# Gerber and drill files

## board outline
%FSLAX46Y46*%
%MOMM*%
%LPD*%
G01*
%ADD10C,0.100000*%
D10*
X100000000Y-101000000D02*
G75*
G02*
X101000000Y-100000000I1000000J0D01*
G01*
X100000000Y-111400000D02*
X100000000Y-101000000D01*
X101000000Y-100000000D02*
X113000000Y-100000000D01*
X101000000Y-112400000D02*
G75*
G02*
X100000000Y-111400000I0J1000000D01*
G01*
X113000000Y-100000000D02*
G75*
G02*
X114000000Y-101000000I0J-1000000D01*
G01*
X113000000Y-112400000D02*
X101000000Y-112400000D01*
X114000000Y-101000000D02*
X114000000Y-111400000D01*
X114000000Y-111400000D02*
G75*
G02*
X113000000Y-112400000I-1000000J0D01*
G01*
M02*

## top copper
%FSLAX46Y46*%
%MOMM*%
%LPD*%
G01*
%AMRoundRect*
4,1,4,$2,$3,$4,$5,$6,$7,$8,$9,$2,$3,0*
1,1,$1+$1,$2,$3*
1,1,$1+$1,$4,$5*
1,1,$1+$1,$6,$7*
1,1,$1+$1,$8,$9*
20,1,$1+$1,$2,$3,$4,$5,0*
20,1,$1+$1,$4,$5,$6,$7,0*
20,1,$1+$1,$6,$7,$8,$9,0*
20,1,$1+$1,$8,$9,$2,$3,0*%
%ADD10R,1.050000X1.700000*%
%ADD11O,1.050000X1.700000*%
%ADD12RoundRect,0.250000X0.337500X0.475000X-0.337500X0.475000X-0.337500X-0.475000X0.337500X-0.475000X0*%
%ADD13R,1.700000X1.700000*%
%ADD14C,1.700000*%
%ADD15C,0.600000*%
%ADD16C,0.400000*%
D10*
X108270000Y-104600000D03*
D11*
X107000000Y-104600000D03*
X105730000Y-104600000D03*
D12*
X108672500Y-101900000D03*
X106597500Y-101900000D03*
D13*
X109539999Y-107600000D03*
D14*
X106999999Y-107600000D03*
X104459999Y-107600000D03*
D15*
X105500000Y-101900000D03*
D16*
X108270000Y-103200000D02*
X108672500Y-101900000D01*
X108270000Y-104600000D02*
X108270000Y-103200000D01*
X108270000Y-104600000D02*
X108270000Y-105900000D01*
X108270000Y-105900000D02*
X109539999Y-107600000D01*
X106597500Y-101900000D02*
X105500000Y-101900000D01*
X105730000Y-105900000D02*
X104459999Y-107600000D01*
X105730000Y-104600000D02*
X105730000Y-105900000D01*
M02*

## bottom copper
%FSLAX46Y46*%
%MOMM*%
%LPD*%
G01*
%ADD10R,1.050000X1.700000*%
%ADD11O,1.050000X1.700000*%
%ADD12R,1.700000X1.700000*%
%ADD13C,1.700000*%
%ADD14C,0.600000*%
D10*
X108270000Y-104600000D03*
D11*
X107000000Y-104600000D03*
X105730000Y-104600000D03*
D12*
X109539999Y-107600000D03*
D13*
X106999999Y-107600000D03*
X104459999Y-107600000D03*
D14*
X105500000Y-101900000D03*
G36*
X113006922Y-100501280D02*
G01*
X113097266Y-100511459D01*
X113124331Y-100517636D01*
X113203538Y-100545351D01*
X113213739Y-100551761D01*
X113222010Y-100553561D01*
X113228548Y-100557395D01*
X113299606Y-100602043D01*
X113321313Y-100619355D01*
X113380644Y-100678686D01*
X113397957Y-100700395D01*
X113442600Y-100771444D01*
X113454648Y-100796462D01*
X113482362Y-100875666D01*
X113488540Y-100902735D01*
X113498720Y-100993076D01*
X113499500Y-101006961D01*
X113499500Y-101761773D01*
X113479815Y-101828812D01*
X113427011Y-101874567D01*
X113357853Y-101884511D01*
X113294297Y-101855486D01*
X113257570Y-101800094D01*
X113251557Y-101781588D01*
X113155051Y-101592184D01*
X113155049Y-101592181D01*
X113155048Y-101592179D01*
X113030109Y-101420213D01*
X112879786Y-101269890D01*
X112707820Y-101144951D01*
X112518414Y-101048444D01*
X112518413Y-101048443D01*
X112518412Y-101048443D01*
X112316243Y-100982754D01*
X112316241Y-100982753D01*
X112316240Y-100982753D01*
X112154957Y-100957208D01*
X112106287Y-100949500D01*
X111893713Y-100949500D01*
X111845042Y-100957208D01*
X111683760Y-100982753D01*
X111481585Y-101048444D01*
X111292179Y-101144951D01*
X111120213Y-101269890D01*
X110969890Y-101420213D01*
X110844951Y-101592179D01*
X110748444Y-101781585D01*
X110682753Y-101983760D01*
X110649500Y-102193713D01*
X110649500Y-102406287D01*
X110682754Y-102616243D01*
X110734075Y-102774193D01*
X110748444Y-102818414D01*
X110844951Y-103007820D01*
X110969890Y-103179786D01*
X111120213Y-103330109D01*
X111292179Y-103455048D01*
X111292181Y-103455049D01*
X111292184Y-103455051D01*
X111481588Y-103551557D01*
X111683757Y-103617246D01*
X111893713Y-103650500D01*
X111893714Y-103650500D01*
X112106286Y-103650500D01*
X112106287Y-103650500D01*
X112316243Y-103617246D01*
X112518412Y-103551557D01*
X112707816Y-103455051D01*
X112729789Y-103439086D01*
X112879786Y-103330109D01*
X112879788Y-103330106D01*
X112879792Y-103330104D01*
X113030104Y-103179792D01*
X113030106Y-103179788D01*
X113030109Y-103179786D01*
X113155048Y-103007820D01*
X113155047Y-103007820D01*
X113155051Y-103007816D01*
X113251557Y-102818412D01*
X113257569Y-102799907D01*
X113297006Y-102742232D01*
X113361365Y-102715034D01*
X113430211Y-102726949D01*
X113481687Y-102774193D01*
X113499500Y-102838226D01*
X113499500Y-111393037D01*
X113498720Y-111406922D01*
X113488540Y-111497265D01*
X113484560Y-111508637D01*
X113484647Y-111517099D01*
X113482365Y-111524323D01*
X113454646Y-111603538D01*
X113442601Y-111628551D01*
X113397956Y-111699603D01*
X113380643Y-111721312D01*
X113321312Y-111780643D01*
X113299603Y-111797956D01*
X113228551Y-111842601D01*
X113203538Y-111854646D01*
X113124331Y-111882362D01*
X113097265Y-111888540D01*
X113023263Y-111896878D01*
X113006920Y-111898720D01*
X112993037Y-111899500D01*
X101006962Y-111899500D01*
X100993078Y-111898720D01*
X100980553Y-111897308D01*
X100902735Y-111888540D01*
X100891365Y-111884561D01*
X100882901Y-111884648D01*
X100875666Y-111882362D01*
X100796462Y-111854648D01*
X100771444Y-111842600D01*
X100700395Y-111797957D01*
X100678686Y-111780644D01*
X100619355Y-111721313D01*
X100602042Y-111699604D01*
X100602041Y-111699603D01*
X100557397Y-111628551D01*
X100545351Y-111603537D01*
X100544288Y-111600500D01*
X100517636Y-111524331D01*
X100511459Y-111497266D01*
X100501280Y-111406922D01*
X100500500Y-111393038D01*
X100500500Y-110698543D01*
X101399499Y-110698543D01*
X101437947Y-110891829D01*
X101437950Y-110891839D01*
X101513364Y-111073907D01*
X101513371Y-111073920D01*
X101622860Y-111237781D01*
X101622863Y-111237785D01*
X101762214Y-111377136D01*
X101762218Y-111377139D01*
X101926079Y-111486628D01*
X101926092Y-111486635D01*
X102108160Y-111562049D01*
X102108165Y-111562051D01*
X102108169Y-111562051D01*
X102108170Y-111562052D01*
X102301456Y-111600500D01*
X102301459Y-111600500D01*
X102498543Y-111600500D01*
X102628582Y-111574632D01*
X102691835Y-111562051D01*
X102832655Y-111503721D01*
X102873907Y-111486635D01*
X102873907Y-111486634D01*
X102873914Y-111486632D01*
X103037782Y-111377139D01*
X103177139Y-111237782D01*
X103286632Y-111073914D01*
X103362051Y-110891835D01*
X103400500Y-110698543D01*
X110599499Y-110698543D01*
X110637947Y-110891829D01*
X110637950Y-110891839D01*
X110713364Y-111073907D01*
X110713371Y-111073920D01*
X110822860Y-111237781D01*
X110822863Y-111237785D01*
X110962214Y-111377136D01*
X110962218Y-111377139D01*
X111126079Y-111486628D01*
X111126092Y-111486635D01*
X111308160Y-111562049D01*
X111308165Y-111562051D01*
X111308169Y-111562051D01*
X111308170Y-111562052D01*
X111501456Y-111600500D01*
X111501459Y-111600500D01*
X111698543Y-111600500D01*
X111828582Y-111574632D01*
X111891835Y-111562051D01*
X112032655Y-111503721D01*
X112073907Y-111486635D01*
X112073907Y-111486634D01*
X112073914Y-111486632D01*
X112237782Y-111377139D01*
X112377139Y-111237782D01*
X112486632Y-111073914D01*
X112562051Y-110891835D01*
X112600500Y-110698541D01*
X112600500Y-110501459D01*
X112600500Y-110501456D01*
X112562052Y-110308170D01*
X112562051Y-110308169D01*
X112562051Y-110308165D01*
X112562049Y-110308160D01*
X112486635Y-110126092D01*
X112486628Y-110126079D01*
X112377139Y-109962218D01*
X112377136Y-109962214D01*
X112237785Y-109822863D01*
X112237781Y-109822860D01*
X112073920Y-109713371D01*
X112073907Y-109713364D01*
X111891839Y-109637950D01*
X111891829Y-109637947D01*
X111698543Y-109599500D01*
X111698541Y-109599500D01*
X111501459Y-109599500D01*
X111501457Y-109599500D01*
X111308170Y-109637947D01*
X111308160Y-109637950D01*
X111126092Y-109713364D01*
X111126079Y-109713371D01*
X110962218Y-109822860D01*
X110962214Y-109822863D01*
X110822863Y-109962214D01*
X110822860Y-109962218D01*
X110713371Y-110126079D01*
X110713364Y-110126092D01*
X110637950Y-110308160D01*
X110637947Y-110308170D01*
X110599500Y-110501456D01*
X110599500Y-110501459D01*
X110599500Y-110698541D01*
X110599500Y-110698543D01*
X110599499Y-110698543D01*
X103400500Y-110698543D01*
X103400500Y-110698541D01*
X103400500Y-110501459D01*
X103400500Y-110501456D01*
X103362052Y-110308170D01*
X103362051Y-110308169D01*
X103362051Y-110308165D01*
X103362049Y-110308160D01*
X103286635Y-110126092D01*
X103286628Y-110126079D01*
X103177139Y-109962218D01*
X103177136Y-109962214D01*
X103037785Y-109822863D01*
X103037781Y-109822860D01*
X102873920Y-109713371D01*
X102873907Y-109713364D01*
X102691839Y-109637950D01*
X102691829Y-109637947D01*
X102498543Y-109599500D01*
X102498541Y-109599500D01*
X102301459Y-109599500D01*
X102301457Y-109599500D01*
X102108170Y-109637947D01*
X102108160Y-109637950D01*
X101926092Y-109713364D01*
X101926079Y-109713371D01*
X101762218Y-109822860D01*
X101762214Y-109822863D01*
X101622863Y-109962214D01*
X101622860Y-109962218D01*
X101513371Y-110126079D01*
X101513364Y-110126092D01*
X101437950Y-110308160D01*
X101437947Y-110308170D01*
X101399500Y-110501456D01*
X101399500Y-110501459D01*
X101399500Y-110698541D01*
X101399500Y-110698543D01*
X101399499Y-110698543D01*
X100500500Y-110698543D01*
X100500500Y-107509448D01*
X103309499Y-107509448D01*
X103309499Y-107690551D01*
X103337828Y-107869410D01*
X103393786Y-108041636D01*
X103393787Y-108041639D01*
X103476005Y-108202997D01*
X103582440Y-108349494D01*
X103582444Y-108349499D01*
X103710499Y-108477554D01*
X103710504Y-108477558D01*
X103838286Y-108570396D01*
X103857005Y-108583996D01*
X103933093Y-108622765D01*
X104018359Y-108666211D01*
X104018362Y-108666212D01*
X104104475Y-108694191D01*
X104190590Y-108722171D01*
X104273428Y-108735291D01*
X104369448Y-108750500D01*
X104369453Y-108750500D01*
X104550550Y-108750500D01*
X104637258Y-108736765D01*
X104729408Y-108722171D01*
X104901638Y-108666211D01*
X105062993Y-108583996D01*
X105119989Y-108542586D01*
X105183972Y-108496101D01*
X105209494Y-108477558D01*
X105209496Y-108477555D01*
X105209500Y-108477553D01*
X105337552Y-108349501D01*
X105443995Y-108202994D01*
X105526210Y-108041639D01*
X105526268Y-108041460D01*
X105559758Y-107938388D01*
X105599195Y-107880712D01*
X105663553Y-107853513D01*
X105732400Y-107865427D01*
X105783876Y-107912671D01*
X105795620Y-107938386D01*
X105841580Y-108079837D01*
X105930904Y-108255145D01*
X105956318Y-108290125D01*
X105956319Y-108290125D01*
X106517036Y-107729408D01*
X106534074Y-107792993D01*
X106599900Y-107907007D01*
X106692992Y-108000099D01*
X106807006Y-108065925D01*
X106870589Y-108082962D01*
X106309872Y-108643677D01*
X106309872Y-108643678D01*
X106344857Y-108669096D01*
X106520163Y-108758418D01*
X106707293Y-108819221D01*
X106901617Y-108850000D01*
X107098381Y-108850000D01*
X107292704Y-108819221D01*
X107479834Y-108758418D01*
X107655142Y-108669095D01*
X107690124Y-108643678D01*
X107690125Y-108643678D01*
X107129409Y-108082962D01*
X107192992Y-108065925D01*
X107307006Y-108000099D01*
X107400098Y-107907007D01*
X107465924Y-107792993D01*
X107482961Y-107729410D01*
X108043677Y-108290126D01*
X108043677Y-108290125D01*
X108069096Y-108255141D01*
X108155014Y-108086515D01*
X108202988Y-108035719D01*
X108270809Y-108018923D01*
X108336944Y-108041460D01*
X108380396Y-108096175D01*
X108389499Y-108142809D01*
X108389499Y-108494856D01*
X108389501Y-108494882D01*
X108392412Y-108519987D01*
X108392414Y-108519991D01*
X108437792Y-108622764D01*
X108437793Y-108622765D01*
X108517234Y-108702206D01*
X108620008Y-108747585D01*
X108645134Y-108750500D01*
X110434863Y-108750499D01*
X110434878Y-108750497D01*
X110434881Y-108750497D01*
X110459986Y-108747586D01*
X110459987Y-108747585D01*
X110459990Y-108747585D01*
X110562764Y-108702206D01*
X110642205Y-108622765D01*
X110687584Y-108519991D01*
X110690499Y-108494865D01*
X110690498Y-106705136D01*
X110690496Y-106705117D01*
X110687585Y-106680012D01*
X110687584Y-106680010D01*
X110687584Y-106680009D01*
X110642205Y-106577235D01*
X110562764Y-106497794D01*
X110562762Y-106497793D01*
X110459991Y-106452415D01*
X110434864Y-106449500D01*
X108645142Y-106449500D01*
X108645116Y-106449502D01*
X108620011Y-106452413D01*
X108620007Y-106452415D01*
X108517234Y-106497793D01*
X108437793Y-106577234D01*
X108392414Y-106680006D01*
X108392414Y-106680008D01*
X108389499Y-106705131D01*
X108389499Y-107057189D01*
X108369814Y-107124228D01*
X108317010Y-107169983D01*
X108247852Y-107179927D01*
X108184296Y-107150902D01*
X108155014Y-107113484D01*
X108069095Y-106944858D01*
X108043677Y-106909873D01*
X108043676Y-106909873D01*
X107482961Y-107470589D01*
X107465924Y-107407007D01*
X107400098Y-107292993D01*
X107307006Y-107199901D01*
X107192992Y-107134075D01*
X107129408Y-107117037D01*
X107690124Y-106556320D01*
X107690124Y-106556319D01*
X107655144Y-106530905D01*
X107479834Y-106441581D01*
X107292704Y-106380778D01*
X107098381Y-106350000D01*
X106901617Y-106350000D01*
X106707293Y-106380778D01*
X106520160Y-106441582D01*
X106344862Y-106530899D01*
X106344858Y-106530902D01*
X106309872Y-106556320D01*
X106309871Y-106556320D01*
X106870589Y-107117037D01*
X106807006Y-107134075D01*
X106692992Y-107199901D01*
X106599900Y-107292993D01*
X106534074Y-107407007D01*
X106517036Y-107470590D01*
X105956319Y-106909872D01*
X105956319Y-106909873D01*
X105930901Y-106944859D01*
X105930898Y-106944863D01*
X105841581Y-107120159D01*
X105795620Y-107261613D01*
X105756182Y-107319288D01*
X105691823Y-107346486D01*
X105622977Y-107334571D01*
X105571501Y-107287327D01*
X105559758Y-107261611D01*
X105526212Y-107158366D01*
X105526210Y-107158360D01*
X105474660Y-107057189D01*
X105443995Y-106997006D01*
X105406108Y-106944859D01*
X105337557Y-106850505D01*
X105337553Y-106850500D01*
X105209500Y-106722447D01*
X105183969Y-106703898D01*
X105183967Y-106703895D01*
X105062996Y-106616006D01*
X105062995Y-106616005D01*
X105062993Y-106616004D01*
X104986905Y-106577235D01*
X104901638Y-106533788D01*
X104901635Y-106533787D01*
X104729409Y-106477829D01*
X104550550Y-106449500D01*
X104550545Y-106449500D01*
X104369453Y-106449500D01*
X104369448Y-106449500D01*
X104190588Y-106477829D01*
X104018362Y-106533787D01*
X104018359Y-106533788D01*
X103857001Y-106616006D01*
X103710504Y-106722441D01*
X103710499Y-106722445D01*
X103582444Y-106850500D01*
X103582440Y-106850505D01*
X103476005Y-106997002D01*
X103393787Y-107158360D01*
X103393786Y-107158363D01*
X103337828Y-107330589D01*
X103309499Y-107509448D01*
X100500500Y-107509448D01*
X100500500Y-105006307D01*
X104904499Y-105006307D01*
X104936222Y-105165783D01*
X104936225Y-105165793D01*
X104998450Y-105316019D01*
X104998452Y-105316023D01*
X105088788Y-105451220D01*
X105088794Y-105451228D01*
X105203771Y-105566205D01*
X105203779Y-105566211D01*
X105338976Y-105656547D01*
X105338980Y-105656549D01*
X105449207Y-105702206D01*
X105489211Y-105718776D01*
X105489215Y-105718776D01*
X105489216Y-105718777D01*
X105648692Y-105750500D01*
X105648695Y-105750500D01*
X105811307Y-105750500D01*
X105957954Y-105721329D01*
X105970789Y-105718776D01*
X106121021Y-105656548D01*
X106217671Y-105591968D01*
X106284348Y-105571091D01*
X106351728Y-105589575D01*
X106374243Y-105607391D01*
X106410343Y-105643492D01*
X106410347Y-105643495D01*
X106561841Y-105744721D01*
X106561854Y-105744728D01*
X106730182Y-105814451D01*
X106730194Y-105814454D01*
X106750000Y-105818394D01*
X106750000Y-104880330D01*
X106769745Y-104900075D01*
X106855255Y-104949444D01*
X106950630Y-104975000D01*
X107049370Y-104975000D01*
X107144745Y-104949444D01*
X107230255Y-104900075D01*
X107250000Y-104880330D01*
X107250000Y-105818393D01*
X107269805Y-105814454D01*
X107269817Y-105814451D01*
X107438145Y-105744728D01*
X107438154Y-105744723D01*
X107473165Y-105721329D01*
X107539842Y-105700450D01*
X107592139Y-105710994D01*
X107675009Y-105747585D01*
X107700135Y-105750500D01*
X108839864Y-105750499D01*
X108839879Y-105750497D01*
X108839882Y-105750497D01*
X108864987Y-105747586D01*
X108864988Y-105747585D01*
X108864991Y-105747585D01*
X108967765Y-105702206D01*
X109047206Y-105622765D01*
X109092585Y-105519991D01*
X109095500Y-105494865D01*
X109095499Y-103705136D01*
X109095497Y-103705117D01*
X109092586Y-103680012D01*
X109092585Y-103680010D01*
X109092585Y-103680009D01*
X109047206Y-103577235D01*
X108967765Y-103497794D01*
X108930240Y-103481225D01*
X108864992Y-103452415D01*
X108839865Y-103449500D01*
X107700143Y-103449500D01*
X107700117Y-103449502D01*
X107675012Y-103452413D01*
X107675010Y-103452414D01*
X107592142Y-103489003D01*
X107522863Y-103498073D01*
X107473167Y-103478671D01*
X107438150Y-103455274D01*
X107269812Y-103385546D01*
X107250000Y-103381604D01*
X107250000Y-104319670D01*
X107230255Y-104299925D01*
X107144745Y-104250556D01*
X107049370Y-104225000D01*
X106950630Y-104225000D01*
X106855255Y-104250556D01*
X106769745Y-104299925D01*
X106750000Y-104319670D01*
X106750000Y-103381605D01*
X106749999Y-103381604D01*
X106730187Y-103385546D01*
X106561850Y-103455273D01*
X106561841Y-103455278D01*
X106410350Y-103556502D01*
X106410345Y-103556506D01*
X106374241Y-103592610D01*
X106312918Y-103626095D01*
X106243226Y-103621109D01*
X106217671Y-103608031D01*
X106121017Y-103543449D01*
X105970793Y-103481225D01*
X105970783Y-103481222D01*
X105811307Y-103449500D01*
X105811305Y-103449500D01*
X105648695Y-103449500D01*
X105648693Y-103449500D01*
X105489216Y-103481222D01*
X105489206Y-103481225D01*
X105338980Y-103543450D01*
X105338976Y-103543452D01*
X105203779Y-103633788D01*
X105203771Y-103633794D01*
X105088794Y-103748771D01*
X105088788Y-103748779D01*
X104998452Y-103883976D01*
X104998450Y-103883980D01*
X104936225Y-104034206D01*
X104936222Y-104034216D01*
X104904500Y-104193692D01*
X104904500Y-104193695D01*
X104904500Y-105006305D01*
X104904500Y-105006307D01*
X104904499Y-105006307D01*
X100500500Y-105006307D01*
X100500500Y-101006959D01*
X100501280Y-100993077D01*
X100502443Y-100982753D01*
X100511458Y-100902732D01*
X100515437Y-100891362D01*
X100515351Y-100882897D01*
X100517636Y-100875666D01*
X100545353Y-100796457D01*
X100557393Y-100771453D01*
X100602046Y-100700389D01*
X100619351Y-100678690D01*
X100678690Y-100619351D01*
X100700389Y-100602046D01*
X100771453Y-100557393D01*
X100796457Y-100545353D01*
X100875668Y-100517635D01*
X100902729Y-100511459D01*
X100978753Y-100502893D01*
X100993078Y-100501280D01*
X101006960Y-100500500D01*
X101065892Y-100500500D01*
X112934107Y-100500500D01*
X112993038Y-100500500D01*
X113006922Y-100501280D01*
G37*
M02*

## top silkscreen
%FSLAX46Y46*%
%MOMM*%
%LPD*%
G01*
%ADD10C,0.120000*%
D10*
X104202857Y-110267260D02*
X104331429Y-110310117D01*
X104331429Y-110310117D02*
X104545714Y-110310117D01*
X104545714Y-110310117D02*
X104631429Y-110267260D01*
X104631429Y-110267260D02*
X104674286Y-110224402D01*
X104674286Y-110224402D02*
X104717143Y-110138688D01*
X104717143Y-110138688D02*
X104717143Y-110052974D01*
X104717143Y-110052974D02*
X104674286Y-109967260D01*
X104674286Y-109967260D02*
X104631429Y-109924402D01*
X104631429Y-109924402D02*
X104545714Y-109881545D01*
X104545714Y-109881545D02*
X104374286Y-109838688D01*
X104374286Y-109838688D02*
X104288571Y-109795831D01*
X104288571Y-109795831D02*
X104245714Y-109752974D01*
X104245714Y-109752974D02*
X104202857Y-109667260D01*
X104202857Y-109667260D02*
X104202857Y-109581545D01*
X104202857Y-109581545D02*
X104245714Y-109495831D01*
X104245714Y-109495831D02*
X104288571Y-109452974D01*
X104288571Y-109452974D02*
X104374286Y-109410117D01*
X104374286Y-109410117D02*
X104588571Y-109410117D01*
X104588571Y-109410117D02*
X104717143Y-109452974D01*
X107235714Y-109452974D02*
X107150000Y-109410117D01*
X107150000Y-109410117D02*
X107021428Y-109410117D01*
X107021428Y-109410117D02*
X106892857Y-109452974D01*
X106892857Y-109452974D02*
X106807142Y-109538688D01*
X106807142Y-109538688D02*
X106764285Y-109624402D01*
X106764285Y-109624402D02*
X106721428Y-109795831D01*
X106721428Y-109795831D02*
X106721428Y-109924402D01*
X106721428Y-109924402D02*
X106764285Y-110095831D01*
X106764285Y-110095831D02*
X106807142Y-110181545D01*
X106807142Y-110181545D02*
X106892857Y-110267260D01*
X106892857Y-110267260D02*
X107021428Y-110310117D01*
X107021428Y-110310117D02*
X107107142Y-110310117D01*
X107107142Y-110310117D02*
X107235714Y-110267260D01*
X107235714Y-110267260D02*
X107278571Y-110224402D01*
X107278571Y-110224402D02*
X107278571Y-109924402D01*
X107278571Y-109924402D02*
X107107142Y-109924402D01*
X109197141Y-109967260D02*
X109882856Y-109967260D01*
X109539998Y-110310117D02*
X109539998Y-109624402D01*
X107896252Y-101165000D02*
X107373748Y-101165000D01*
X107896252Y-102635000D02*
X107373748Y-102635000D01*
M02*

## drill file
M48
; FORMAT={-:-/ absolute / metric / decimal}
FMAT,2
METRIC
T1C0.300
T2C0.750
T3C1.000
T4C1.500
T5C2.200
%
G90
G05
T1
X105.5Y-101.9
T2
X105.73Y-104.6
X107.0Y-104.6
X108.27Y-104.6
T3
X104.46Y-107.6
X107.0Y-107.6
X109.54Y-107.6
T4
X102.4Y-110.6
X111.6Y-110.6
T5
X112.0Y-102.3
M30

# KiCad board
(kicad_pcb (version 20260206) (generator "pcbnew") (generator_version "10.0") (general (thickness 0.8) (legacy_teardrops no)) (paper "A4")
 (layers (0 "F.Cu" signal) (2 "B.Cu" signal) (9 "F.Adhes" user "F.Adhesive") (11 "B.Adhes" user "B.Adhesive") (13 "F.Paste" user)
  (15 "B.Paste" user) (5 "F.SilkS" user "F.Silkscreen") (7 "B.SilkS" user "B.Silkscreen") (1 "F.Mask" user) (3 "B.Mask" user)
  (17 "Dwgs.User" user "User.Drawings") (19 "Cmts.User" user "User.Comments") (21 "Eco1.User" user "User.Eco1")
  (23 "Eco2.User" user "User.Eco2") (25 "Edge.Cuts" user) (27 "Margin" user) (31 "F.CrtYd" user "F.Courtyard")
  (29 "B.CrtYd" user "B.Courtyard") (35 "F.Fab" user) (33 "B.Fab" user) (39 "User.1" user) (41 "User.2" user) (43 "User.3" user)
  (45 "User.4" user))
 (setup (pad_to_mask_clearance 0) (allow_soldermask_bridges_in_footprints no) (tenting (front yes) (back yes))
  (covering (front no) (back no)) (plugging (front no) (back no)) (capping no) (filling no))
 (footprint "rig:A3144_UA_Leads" (layer "F.Cu") (at 107 104.6)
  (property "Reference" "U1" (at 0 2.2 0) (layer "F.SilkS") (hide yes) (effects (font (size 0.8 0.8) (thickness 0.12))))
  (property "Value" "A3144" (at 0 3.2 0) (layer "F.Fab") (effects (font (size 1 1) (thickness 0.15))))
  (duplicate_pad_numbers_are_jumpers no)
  (pad "1" thru_hole rect (at 1.27 0) (size 1.05 1.7) (drill 0.75) (layers "*.Cu" "*.Mask") (remove_unused_layers no) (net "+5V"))
  (pad "2" thru_hole oval (at 0 0) (size 1.05 1.7) (drill 0.75) (layers "*.Cu" "*.Mask") (remove_unused_layers no) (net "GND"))
  (pad "3" thru_hole oval (at -1.27 0) (size 1.05 1.7) (drill 0.75) (layers "*.Cu" "*.Mask") (remove_unused_layers no) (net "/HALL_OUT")))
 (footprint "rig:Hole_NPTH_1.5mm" (layer "F.Cu") (at 102.4 110.6)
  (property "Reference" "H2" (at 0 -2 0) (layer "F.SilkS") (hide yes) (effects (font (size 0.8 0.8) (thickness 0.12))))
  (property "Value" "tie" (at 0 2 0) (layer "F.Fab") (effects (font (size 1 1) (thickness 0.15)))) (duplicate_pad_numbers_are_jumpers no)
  (pad "" np_thru_hole circle (at 0 0) (size 1.5 1.5) (drill 1.5) (layers "*.Cu" "*.Mask")))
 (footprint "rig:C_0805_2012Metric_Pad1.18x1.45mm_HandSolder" (layer "F.Cu") (at 107.635 101.9 180)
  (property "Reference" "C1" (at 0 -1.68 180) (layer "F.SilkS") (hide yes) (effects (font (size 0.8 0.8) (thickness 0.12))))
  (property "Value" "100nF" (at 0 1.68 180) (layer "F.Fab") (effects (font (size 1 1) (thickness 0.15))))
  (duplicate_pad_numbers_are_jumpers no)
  (fp_line (start -0.261252 0.735) (end 0.261252 0.735) (stroke (width 0.12) (type solid)) (layer "F.SilkS"))
  (fp_line (start -0.261252 -0.735) (end 0.261252 -0.735) (stroke (width 0.12) (type solid)) (layer "F.SilkS"))
  (pad "1" smd roundrect (at -1.0375 0 180) (size 1.175 1.45) (layers "F.Cu" "F.Mask" "F.Paste") (roundrect_rratio 0.212766) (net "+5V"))
  (pad "2" smd roundrect (at 1.0375 0 180) (size 1.175 1.45) (layers "F.Cu" "F.Mask" "F.Paste") (roundrect_rratio 0.212766) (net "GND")))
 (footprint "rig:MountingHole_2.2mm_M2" (layer "F.Cu") (at 112 102.3)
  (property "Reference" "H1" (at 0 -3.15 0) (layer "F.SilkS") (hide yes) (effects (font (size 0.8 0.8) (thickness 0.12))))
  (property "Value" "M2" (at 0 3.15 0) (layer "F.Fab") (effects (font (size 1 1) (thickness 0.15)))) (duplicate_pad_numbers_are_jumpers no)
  (pad "" np_thru_hole circle (at 0 0) (size 2.2 2.2) (drill 2.2) (layers "*.Cu" "*.Mask")))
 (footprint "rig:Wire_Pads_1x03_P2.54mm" (layer "F.Cu") (at 109.539999 107.6 180)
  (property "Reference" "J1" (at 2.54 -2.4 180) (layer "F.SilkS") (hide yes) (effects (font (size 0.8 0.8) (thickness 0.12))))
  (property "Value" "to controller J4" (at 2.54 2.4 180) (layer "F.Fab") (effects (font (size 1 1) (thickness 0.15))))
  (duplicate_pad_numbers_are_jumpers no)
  (pad "1" thru_hole rect (at 0 0 180) (size 1.7 1.7) (drill 1) (layers "*.Cu" "*.Mask") (remove_unused_layers no) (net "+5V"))
  (pad "2" thru_hole circle (at 2.54 0 180) (size 1.7 1.7) (drill 1) (layers "*.Cu" "*.Mask") (remove_unused_layers no) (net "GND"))
  (pad "3" thru_hole circle (at 5.08 0 180) (size 1.7 1.7) (drill 1) (layers "*.Cu" "*.Mask") (remove_unused_layers no) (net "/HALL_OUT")))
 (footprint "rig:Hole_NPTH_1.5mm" (layer "F.Cu") (at 111.6 110.6)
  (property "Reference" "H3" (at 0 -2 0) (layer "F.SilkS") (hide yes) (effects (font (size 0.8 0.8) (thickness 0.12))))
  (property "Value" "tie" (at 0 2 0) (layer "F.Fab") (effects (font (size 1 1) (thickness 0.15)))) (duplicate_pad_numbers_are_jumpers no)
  (pad "" np_thru_hole circle (at 0 0) (size 1.5 1.5) (drill 1.5) (layers "*.Cu" "*.Mask")))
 (gr_arc (start 100 101) (mid 100.292893 100.292893) (end 101 100) (stroke (width 0.1) (type default)) (layer "Edge.Cuts"))
 (gr_line (start 100 111.4) (end 100 101) (stroke (width 0.1) (type default)) (layer "Edge.Cuts"))
 (gr_line (start 101 100) (end 113 100) (stroke (width 0.1) (type default)) (layer "Edge.Cuts"))
 (gr_arc (start 101 112.4) (mid 100.292893 112.107106) (end 100 111.4) (stroke (width 0.1) (type default)) (layer "Edge.Cuts"))
 (gr_arc (start 113 100) (mid 113.707106 100.292893) (end 114 101) (stroke (width 0.1) (type default)) (layer "Edge.Cuts"))
 (gr_line (start 113 112.4) (end 101 112.4) (stroke (width 0.1) (type default)) (layer "Edge.Cuts"))
 (gr_line (start 114 101) (end 114 111.4) (stroke (width 0.1) (type default)) (layer "Edge.Cuts"))
 (gr_arc (start 114 111.4) (mid 113.707106 112.107106) (end 113 112.4) (stroke (width 0.1) (type default)) (layer "Edge.Cuts"))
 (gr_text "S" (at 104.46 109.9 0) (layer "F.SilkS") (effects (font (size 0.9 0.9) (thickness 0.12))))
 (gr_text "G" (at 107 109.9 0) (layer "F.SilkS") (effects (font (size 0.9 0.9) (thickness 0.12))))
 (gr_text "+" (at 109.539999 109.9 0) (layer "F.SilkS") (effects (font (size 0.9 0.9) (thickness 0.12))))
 (segment (start 108.27 103.2) (end 108.6725 101.9) (width 0.4) (layer "F.Cu") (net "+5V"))
 (segment (start 108.27 104.6) (end 108.27 103.2) (width 0.4) (layer "F.Cu") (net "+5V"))
 (segment (start 108.27 104.6) (end 108.27 105.9) (width 0.4) (layer "F.Cu") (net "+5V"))
 (segment (start 108.27 105.9) (end 109.539999 107.6) (width 0.4) (layer "F.Cu") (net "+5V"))
 (segment (start 106.5975 101.9) (end 105.5 101.9) (width 0.4) (layer "F.Cu") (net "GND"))
 (via (at 105.5 101.9) (size 0.6) (drill 0.3) (layers "F.Cu" "B.Cu") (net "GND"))
 (segment (start 105.73 105.9) (end 104.459999 107.6) (width 0.4) (layer "F.Cu") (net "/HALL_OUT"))
 (segment (start 105.73 104.6) (end 105.73 105.9) (width 0.4) (layer "F.Cu") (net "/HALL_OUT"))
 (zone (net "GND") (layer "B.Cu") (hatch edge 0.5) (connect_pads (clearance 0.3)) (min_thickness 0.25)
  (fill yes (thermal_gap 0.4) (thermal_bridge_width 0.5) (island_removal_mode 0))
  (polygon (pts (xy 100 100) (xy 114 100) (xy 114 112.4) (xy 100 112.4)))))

